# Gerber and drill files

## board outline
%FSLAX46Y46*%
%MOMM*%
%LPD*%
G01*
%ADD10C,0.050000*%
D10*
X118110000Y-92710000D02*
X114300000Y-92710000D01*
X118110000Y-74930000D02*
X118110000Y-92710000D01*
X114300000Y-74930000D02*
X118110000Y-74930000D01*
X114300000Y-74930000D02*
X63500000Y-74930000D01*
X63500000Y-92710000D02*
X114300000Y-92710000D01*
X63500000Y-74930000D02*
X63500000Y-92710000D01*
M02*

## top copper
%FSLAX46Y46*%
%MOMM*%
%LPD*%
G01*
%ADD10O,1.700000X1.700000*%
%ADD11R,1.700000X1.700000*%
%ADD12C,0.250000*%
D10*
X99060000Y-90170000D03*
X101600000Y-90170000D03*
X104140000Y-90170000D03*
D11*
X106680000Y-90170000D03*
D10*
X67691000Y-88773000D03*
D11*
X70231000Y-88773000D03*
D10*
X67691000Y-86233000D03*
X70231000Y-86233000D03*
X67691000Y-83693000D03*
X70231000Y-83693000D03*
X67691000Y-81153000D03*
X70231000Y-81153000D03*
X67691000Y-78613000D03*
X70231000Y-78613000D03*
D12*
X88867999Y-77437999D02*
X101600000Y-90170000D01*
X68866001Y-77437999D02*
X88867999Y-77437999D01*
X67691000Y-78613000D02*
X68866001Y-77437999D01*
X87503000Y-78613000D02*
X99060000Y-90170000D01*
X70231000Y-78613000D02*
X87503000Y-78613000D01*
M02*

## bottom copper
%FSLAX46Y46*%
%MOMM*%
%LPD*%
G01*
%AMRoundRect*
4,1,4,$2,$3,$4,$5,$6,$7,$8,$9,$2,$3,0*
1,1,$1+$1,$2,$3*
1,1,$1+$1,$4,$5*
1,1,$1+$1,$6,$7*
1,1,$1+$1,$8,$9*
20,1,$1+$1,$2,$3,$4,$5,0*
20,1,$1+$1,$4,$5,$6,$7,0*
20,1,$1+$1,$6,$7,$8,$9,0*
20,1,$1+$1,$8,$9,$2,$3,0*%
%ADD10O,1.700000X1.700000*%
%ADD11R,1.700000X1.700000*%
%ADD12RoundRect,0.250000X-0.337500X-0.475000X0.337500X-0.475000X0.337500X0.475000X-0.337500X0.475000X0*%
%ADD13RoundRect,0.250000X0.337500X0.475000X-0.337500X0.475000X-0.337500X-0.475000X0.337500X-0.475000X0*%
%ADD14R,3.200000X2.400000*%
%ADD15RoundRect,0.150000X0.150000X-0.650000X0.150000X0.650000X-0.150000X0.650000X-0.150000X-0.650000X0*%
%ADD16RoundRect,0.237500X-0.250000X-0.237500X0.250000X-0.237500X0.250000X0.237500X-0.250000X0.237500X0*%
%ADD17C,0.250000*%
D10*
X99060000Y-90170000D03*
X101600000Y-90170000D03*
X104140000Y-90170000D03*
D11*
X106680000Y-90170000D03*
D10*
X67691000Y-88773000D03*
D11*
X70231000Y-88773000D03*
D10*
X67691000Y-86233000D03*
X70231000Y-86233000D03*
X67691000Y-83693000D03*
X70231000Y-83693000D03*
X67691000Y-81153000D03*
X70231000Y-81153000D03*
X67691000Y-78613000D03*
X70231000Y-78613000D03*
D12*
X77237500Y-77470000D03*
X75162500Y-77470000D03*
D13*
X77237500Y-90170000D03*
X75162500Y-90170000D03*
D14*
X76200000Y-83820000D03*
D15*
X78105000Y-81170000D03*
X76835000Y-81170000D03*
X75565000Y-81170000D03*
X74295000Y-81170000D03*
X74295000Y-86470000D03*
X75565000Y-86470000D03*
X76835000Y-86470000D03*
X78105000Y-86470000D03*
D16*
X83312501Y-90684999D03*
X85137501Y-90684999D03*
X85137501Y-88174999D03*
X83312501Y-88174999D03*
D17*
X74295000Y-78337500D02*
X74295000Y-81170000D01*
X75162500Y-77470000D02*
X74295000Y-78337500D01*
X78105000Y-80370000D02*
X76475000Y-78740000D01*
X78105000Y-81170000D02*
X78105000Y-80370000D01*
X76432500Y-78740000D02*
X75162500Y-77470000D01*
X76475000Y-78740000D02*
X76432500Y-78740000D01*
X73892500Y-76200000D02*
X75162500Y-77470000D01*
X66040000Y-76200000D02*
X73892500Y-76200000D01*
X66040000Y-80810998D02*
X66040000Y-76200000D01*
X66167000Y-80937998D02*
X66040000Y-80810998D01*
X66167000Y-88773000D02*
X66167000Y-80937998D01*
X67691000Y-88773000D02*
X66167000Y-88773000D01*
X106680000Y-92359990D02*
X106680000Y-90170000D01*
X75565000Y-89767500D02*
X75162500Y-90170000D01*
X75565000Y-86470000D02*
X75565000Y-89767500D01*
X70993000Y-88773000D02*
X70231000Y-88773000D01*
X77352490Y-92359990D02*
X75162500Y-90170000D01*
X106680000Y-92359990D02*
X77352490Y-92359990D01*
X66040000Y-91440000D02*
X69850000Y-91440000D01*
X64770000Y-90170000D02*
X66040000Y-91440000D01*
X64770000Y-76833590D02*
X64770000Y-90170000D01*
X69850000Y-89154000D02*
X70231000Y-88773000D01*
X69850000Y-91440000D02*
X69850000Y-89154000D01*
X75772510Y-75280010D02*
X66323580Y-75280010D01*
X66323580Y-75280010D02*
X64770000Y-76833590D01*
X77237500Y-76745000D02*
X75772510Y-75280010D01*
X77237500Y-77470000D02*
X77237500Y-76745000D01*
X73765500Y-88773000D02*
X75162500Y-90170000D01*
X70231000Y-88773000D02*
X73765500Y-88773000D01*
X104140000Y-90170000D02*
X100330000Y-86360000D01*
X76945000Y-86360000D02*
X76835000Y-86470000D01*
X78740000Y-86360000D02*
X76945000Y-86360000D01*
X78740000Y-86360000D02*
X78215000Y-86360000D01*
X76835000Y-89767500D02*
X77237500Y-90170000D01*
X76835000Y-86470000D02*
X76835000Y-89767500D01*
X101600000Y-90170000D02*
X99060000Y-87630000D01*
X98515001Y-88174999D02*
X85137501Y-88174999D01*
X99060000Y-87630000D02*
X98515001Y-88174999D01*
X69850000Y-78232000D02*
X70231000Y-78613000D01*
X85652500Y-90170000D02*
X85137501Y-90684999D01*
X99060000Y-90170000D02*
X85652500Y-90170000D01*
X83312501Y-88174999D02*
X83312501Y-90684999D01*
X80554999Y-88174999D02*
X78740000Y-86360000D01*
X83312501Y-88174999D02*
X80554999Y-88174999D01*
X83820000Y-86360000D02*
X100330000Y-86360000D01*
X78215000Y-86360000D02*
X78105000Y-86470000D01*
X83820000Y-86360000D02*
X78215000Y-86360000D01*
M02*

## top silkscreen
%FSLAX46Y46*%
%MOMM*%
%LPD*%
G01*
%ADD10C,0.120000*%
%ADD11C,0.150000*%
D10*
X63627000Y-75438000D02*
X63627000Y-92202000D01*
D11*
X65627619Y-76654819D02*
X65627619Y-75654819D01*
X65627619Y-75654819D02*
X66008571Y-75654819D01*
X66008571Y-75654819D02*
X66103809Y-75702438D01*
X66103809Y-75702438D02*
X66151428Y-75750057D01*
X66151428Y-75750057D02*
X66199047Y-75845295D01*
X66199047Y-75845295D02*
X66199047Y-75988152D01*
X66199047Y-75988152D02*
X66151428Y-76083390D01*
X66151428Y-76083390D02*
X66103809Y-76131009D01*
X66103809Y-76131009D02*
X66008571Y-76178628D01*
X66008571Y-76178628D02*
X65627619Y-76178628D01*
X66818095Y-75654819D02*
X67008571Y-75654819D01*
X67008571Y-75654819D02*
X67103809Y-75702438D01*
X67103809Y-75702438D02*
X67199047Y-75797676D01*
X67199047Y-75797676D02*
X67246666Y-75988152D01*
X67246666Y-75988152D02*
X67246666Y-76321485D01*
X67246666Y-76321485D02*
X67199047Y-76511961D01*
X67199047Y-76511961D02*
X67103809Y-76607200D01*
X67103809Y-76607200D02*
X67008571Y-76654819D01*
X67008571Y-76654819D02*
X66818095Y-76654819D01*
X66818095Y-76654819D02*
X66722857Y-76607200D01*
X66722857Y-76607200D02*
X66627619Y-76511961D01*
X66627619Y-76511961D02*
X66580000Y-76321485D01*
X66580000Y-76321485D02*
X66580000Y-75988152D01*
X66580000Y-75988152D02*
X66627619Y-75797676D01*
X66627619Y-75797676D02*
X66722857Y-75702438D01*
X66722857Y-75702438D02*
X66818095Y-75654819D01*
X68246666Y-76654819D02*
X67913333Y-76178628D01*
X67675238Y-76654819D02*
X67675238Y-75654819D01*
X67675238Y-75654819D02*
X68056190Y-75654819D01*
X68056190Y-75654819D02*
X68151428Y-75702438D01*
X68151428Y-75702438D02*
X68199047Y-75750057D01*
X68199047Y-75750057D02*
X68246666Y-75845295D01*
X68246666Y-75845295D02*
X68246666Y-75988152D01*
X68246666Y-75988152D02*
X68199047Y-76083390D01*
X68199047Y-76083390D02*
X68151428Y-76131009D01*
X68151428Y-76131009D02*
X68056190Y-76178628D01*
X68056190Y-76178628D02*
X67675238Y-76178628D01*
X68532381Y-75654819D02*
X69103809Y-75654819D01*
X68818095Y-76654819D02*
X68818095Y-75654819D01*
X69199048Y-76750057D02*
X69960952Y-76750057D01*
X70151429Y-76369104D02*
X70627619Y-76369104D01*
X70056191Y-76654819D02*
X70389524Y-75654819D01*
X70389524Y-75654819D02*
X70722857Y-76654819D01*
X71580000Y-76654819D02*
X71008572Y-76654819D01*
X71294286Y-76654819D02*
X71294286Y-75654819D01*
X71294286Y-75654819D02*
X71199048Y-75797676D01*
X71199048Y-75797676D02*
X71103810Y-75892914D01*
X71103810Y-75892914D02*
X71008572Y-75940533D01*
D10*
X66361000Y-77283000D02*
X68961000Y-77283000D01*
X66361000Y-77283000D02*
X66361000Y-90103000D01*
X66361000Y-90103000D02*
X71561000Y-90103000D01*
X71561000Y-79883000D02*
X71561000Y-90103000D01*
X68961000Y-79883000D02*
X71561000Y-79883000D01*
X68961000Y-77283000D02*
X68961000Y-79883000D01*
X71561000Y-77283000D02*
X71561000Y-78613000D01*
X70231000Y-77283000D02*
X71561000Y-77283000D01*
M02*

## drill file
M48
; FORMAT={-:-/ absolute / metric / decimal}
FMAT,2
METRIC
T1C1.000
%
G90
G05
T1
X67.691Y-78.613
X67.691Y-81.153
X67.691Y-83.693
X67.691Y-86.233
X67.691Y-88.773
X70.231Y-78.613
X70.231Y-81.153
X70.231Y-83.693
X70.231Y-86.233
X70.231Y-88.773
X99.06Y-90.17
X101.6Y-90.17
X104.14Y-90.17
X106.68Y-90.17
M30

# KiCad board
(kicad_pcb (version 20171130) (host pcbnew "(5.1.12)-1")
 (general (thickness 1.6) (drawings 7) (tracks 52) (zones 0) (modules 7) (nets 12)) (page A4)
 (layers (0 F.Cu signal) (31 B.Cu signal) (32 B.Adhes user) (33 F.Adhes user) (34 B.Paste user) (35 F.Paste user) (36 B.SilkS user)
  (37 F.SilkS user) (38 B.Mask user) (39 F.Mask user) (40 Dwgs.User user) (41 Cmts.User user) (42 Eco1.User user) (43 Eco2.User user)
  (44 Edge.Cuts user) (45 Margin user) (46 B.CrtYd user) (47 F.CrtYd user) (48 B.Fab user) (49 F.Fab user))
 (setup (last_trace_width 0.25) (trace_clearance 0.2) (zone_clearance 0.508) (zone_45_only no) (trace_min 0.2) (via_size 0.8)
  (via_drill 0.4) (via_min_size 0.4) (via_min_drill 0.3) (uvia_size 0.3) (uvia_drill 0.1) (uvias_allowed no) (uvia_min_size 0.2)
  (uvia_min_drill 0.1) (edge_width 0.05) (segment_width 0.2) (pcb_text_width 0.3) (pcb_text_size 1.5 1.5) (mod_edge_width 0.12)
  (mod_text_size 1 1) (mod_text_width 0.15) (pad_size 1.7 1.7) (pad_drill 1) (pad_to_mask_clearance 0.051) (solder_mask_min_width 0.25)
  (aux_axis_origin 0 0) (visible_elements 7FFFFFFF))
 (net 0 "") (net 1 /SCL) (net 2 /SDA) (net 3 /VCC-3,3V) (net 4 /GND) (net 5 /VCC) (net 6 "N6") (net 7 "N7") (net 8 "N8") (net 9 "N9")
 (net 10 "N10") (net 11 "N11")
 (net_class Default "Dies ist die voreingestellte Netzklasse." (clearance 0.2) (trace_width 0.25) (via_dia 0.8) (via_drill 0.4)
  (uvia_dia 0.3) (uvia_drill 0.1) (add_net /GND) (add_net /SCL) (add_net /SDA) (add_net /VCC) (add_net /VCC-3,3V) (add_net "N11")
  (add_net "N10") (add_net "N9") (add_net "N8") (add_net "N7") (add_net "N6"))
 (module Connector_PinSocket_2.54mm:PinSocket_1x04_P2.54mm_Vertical (layer B.Cu) (at 106.68 90.17 90)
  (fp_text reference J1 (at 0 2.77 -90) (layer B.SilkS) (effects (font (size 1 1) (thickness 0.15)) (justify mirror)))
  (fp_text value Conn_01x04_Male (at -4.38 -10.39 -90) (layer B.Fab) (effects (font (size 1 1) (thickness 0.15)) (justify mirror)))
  (pad 4 thru_hole oval (at 0 -7.62 90) (size 1.7 1.7) (drill 1) (layers *.Cu *.Mask) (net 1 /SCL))
  (pad 3 thru_hole oval (at 0 -5.08 90) (size 1.7 1.7) (drill 1) (layers *.Cu *.Mask) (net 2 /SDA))
  (pad 2 thru_hole oval (at 0 -2.54 90) (size 1.7 1.7) (drill 1) (layers *.Cu *.Mask) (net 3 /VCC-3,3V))
  (pad 1 thru_hole rect (at 0 0 90) (size 1.7 1.7) (drill 1) (layers *.Cu *.Mask) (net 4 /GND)))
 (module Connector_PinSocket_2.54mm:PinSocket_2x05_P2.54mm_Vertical (layer F.Cu) (at 70.231 78.613)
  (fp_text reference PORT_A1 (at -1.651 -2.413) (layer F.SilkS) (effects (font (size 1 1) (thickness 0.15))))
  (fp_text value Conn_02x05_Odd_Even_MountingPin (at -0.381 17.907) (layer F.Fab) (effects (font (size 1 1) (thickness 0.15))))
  (fp_line (start -3.87 -1.33) (end -1.27 -1.33) (layer F.SilkS) (width 0.12))
  (fp_line (start -3.87 -1.33) (end -3.87 11.49) (layer F.SilkS) (width 0.12))
  (fp_line (start -3.87 11.49) (end 1.33 11.49) (layer F.SilkS) (width 0.12))
  (fp_line (start 1.33 1.27) (end 1.33 11.49) (layer F.SilkS) (width 0.12))
  (fp_line (start -1.27 1.27) (end 1.33 1.27) (layer F.SilkS) (width 0.12))
  (fp_line (start -1.27 -1.33) (end -1.27 1.27) (layer F.SilkS) (width 0.12))
  (fp_line (start 1.33 -1.33) (end 1.33 0) (layer F.SilkS) (width 0.12))
  (fp_line (start 0 -1.33) (end 1.33 -1.33) (layer F.SilkS) (width 0.12))
  (pad 10 thru_hole oval (at -2.54 10.16) (size 1.7 1.7) (drill 1) (layers *.Cu *.Mask) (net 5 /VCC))
  (pad 9 thru_hole rect (at 0 10.16) (size 1.7 1.7) (drill 1) (layers *.Cu *.Mask) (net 4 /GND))
  (pad 8 thru_hole oval (at -2.54 7.62) (size 1.7 1.7) (drill 1) (layers *.Cu *.Mask) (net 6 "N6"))
  (pad 7 thru_hole oval (at 0 7.62) (size 1.7 1.7) (drill 1) (layers *.Cu *.Mask) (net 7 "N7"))
  (pad 6 thru_hole oval (at -2.54 5.08) (size 1.7 1.7) (drill 1) (layers *.Cu *.Mask) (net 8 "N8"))
  (pad 5 thru_hole oval (at 0 5.08) (size 1.7 1.7) (drill 1) (layers *.Cu *.Mask) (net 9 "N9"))
  (pad 4 thru_hole oval (at -2.54 2.54) (size 1.7 1.7) (drill 1) (layers *.Cu *.Mask) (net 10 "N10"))
  (pad 3 thru_hole oval (at 0 2.54) (size 1.7 1.7) (drill 1) (layers *.Cu *.Mask) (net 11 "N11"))
  (pad 2 thru_hole oval (at -2.54 0) (size 1.7 1.7) (drill 1) (layers *.Cu *.Mask) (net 2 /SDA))
  (pad 1 thru_hole oval (at 0 0) (size 1.7 1.7) (drill 1) (layers *.Cu *.Mask) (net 1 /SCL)))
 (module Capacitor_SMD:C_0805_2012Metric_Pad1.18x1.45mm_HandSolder (layer B.Cu) (at 76.2 77.47)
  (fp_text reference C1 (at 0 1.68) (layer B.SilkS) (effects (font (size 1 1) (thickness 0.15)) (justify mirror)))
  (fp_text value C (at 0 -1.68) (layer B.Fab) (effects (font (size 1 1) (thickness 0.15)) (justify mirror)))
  (pad 2 smd roundrect (at 1.0375 0) (size 1.175 1.45) (layers B.Cu B.Paste B.Mask) (roundrect_rratio 0.212766) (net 4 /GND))
  (pad 1 smd roundrect (at -1.0375 0) (size 1.175 1.45) (layers B.Cu B.Paste B.Mask) (roundrect_rratio 0.212766) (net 5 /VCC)))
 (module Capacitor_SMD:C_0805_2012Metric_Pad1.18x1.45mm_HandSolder (layer B.Cu) (at 76.2 90.17 180)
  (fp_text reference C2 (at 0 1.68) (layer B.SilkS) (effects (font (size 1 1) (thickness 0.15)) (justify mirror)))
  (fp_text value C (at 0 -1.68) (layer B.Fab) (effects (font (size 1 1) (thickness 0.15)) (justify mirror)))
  (pad 1 smd roundrect (at -1.0375 0 180) (size 1.175 1.45) (layers B.Cu B.Paste B.Mask) (roundrect_rratio 0.212766) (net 3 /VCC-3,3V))
  (pad 2 smd roundrect (at 1.0375 0 180) (size 1.175 1.45) (layers B.Cu B.Paste B.Mask) (roundrect_rratio 0.212766) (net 4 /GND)))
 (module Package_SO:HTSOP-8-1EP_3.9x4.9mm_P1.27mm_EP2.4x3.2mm (layer B.Cu) (at 76.2 83.82 90)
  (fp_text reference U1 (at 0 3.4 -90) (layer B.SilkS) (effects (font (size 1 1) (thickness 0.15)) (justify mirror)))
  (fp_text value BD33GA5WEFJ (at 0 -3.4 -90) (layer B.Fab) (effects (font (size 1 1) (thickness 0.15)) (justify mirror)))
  (pad "" smd roundrect (at 0.6 -0.8 90) (size 0.97 1.29) (layers B.Paste) (roundrect_rratio 0.25))
  (pad "" smd roundrect (at 0.6 0.8 90) (size 0.97 1.29) (layers B.Paste) (roundrect_rratio 0.25))
  (pad "" smd roundrect (at -0.6 -0.8 90) (size 0.97 1.29) (layers B.Paste) (roundrect_rratio 0.25))
  (pad "" smd roundrect (at -0.6 0.8 90) (size 0.97 1.29) (layers B.Paste) (roundrect_rratio 0.25))
  (pad 9 smd rect (at 0 0 90) (size 2.4 3.2) (layers B.Cu B.Mask) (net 4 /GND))
  (pad 8 smd roundrect (at 2.65 1.905 90) (size 1.6 0.6) (layers B.Cu B.Paste B.Mask) (roundrect_rratio 0.25) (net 5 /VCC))
  (pad 7 smd roundrect (at 2.65 0.635 90) (size 1.6 0.6) (layers B.Cu B.Paste B.Mask) (roundrect_rratio 0.25) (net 4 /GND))
  (pad 6 smd roundrect (at 2.65 -0.635 90) (size 1.6 0.6) (layers B.Cu B.Paste B.Mask) (roundrect_rratio 0.25) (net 4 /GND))
  (pad 5 smd roundrect (at 2.65 -1.905 90) (size 1.6 0.6) (layers B.Cu B.Paste B.Mask) (roundrect_rratio 0.25) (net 5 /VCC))
  (pad 4 smd roundrect (at -2.65 -1.905 90) (size 1.6 0.6) (layers B.Cu B.Paste B.Mask) (roundrect_rratio 0.25) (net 4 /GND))
  (pad 3 smd roundrect (at -2.65 -0.635 90) (size 1.6 0.6) (layers B.Cu B.Paste B.Mask) (roundrect_rratio 0.25) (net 4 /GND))
  (pad 2 smd roundrect (at -2.65 0.635 90) (size 1.6 0.6) (layers B.Cu B.Paste B.Mask) (roundrect_rratio 0.25) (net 3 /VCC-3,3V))
  (pad 1 smd roundrect (at -2.65 1.905 90) (size 1.6 0.6) (layers B.Cu B.Paste B.Mask) (roundrect_rratio 0.25) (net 3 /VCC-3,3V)))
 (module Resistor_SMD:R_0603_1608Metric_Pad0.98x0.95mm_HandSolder (layer B.Cu) (at 84.225001 90.684999)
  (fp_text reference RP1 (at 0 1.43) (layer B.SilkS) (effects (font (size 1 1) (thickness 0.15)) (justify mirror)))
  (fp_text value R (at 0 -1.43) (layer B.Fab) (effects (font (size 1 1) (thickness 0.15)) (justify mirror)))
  (pad 1 smd roundrect (at -0.9125 0) (size 0.975 0.95) (layers B.Cu B.Paste B.Mask) (roundrect_rratio 0.25) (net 3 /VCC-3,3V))
  (pad 2 smd roundrect (at 0.9125 0) (size 0.975 0.95) (layers B.Cu B.Paste B.Mask) (roundrect_rratio 0.25) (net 1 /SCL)))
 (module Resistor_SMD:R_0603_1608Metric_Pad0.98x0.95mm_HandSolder (layer B.Cu) (at 84.225001 88.174999)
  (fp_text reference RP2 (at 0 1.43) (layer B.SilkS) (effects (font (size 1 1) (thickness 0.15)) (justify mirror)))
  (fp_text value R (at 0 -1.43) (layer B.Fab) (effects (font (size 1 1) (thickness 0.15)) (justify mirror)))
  (pad 2 smd roundrect (at 0.9125 0) (size 0.975 0.95) (layers B.Cu B.Paste B.Mask) (roundrect_rratio 0.25) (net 2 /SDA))
  (pad 1 smd roundrect (at -0.9125 0) (size 0.975 0.95) (layers B.Cu B.Paste B.Mask) (roundrect_rratio 0.25) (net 3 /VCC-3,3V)))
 (gr_line (start 118.11 92.71) (end 114.3 92.71) (layer Edge.Cuts) (width 0.05))
 (gr_line (start 118.11 74.93) (end 118.11 92.71) (layer Edge.Cuts) (width 0.05))
 (gr_line (start 114.3 74.93) (end 118.11 74.93) (layer Edge.Cuts) (width 0.05))
 (gr_line (start 114.3 74.93) (end 63.5 74.93) (layer Edge.Cuts) (width 0.05))
 (gr_line (start 63.5 92.71) (end 114.3 92.71) (layer Edge.Cuts) (width 0.05))
 (gr_line (start 63.5 74.93) (end 63.5 92.71) (layer Edge.Cuts) (width 0.05))
 (gr_line (start 63.627 75.438) (end 63.627 92.202) (layer F.SilkS) (width 0.12))
 (segment (start 74.295 78.3375) (end 74.295 81.17) (width 0.25) (layer B.Cu) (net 5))
 (segment (start 75.1625 77.47) (end 74.295 78.3375) (width 0.25) (layer B.Cu) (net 5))
 (segment (start 78.105 80.37) (end 76.475 78.74) (width 0.25) (layer B.Cu) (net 5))
 (segment (start 78.105 81.17) (end 78.105 80.37) (width 0.25) (layer B.Cu) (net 5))
 (segment (start 76.4325 78.74) (end 75.1625 77.47) (width 0.25) (layer B.Cu) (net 5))
 (segment (start 76.475 78.74) (end 76.4325 78.74) (width 0.25) (layer B.Cu) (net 5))
 (segment (start 73.8925 76.2) (end 75.1625 77.47) (width 0.25) (layer B.Cu) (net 5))
 (segment (start 66.04 76.2) (end 73.8925 76.2) (width 0.25) (layer B.Cu) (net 5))
 (segment (start 66.04 80.810998) (end 66.04 76.2) (width 0.25) (layer B.Cu) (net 5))
 (segment (start 66.167 80.937998) (end 66.04 80.810998) (width 0.25) (layer B.Cu) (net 5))
 (segment (start 66.167 88.773) (end 66.167 80.937998) (width 0.25) (layer B.Cu) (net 5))
 (segment (start 67.691 88.773) (end 66.167 88.773) (width 0.25) (layer B.Cu) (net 5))
 (segment (start 106.68 92.35999) (end 106.68 90.17) (width 0.25) (layer B.Cu) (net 4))
 (segment (start 75.565 89.7675) (end 75.1625 90.17) (width 0.25) (layer B.Cu) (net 4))
 (segment (start 75.565 86.47) (end 75.565 89.7675) (width 0.25) (layer B.Cu) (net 4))
 (segment (start 70.993 88.773) (end 70.231 88.773) (width 0.25) (layer B.Cu) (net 4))
 (segment (start 77.35249 92.35999) (end 75.1625 90.17) (width 0.25) (layer B.Cu) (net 4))
 (segment (start 106.68 92.35999) (end 77.35249 92.35999) (width 0.25) (layer B.Cu) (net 4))
 (segment (start 66.04 91.44) (end 69.85 91.44) (width 0.25) (layer B.Cu) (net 4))
 (segment (start 64.77 90.17) (end 66.04 91.44) (width 0.25) (layer B.Cu) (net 4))
 (segment (start 64.77 76.83359) (end 64.77 90.17) (width 0.25) (layer B.Cu) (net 4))
 (segment (start 69.85 89.154) (end 70.231 88.773) (width 0.25) (layer B.Cu) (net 4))
 (segment (start 69.85 91.44) (end 69.85 89.154) (width 0.25) (layer B.Cu) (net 4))
 (segment (start 75.77251 75.28001) (end 66.32358 75.28001) (width 0.25) (layer B.Cu) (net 4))
 (segment (start 66.32358 75.28001) (end 64.77 76.83359) (width 0.25) (layer B.Cu) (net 4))
 (segment (start 77.2375 76.745) (end 75.77251 75.28001) (width 0.25) (layer B.Cu) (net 4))
 (segment (start 77.2375 77.47) (end 77.2375 76.745) (width 0.25) (layer B.Cu) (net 4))
 (segment (start 73.7655 88.773) (end 75.1625 90.17) (width 0.25) (layer B.Cu) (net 4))
 (segment (start 70.231 88.773) (end 73.7655 88.773) (width 0.25) (layer B.Cu) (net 4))
 (segment (start 104.14 90.17) (end 100.33 86.36) (width 0.25) (layer B.Cu) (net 3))
 (segment (start 76.945 86.36) (end 76.835 86.47) (width 0.25) (layer B.Cu) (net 3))
 (segment (start 78.74 86.36) (end 76.945 86.36) (width 0.25) (layer B.Cu) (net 3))
 (segment (start 78.74 86.36) (end 78.215 86.36) (width 0.25) (layer B.Cu) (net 3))
 (segment (start 76.835 89.7675) (end 77.2375 90.17) (width 0.25) (layer B.Cu) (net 3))
 (segment (start 76.835 86.47) (end 76.835 89.7675) (width 0.25) (layer B.Cu) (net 3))
 (segment (start 88.867999 77.437999) (end 101.6 90.17) (width 0.25) (layer F.Cu) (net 2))
 (segment (start 68.866001 77.437999) (end 88.867999 77.437999) (width 0.25) (layer F.Cu) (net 2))
 (segment (start 67.691 78.613) (end 68.866001 77.437999) (width 0.25) (layer F.Cu) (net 2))
 (segment (start 101.6 90.17) (end 99.06 87.63) (width 0.25) (layer B.Cu) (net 2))
 (segment (start 98.515001 88.174999) (end 85.137501 88.174999) (width 0.25) (layer B.Cu) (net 2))
 (segment (start 99.06 87.63) (end 98.515001 88.174999) (width 0.25) (layer B.Cu) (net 2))
 (segment (start 69.85 78.232) (end 70.231 78.613) (width 0.25) (layer B.Cu) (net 1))
 (segment (start 87.503 78.613) (end 99.06 90.17) (width 0.25) (layer F.Cu) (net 1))
 (segment (start 70.231 78.613) (end 87.503 78.613) (width 0.25) (layer F.Cu) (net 1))
 (segment (start 85.6525 90.17) (end 85.137501 90.684999) (width 0.25) (layer B.Cu) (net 1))
 (segment (start 99.06 90.17) (end 85.6525 90.17) (width 0.25) (layer B.Cu) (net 1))
 (segment (start 83.312501 88.174999) (end 83.312501 90.684999) (width 0.25) (layer B.Cu) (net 3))
 (segment (start 80.554999 88.174999) (end 78.74 86.36) (width 0.25) (layer B.Cu) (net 3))
 (segment (start 83.312501 88.174999) (end 80.554999 88.174999) (width 0.25) (layer B.Cu) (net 3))
 (segment (start 83.82 86.36) (end 100.33 86.36) (width 0.25) (layer B.Cu) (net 3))
 (segment (start 78.215 86.36) (end 78.105 86.47) (width 0.25) (layer B.Cu) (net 3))
 (segment (start 83.82 86.36) (end 78.215 86.36) (width 0.25) (layer B.Cu) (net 3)))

